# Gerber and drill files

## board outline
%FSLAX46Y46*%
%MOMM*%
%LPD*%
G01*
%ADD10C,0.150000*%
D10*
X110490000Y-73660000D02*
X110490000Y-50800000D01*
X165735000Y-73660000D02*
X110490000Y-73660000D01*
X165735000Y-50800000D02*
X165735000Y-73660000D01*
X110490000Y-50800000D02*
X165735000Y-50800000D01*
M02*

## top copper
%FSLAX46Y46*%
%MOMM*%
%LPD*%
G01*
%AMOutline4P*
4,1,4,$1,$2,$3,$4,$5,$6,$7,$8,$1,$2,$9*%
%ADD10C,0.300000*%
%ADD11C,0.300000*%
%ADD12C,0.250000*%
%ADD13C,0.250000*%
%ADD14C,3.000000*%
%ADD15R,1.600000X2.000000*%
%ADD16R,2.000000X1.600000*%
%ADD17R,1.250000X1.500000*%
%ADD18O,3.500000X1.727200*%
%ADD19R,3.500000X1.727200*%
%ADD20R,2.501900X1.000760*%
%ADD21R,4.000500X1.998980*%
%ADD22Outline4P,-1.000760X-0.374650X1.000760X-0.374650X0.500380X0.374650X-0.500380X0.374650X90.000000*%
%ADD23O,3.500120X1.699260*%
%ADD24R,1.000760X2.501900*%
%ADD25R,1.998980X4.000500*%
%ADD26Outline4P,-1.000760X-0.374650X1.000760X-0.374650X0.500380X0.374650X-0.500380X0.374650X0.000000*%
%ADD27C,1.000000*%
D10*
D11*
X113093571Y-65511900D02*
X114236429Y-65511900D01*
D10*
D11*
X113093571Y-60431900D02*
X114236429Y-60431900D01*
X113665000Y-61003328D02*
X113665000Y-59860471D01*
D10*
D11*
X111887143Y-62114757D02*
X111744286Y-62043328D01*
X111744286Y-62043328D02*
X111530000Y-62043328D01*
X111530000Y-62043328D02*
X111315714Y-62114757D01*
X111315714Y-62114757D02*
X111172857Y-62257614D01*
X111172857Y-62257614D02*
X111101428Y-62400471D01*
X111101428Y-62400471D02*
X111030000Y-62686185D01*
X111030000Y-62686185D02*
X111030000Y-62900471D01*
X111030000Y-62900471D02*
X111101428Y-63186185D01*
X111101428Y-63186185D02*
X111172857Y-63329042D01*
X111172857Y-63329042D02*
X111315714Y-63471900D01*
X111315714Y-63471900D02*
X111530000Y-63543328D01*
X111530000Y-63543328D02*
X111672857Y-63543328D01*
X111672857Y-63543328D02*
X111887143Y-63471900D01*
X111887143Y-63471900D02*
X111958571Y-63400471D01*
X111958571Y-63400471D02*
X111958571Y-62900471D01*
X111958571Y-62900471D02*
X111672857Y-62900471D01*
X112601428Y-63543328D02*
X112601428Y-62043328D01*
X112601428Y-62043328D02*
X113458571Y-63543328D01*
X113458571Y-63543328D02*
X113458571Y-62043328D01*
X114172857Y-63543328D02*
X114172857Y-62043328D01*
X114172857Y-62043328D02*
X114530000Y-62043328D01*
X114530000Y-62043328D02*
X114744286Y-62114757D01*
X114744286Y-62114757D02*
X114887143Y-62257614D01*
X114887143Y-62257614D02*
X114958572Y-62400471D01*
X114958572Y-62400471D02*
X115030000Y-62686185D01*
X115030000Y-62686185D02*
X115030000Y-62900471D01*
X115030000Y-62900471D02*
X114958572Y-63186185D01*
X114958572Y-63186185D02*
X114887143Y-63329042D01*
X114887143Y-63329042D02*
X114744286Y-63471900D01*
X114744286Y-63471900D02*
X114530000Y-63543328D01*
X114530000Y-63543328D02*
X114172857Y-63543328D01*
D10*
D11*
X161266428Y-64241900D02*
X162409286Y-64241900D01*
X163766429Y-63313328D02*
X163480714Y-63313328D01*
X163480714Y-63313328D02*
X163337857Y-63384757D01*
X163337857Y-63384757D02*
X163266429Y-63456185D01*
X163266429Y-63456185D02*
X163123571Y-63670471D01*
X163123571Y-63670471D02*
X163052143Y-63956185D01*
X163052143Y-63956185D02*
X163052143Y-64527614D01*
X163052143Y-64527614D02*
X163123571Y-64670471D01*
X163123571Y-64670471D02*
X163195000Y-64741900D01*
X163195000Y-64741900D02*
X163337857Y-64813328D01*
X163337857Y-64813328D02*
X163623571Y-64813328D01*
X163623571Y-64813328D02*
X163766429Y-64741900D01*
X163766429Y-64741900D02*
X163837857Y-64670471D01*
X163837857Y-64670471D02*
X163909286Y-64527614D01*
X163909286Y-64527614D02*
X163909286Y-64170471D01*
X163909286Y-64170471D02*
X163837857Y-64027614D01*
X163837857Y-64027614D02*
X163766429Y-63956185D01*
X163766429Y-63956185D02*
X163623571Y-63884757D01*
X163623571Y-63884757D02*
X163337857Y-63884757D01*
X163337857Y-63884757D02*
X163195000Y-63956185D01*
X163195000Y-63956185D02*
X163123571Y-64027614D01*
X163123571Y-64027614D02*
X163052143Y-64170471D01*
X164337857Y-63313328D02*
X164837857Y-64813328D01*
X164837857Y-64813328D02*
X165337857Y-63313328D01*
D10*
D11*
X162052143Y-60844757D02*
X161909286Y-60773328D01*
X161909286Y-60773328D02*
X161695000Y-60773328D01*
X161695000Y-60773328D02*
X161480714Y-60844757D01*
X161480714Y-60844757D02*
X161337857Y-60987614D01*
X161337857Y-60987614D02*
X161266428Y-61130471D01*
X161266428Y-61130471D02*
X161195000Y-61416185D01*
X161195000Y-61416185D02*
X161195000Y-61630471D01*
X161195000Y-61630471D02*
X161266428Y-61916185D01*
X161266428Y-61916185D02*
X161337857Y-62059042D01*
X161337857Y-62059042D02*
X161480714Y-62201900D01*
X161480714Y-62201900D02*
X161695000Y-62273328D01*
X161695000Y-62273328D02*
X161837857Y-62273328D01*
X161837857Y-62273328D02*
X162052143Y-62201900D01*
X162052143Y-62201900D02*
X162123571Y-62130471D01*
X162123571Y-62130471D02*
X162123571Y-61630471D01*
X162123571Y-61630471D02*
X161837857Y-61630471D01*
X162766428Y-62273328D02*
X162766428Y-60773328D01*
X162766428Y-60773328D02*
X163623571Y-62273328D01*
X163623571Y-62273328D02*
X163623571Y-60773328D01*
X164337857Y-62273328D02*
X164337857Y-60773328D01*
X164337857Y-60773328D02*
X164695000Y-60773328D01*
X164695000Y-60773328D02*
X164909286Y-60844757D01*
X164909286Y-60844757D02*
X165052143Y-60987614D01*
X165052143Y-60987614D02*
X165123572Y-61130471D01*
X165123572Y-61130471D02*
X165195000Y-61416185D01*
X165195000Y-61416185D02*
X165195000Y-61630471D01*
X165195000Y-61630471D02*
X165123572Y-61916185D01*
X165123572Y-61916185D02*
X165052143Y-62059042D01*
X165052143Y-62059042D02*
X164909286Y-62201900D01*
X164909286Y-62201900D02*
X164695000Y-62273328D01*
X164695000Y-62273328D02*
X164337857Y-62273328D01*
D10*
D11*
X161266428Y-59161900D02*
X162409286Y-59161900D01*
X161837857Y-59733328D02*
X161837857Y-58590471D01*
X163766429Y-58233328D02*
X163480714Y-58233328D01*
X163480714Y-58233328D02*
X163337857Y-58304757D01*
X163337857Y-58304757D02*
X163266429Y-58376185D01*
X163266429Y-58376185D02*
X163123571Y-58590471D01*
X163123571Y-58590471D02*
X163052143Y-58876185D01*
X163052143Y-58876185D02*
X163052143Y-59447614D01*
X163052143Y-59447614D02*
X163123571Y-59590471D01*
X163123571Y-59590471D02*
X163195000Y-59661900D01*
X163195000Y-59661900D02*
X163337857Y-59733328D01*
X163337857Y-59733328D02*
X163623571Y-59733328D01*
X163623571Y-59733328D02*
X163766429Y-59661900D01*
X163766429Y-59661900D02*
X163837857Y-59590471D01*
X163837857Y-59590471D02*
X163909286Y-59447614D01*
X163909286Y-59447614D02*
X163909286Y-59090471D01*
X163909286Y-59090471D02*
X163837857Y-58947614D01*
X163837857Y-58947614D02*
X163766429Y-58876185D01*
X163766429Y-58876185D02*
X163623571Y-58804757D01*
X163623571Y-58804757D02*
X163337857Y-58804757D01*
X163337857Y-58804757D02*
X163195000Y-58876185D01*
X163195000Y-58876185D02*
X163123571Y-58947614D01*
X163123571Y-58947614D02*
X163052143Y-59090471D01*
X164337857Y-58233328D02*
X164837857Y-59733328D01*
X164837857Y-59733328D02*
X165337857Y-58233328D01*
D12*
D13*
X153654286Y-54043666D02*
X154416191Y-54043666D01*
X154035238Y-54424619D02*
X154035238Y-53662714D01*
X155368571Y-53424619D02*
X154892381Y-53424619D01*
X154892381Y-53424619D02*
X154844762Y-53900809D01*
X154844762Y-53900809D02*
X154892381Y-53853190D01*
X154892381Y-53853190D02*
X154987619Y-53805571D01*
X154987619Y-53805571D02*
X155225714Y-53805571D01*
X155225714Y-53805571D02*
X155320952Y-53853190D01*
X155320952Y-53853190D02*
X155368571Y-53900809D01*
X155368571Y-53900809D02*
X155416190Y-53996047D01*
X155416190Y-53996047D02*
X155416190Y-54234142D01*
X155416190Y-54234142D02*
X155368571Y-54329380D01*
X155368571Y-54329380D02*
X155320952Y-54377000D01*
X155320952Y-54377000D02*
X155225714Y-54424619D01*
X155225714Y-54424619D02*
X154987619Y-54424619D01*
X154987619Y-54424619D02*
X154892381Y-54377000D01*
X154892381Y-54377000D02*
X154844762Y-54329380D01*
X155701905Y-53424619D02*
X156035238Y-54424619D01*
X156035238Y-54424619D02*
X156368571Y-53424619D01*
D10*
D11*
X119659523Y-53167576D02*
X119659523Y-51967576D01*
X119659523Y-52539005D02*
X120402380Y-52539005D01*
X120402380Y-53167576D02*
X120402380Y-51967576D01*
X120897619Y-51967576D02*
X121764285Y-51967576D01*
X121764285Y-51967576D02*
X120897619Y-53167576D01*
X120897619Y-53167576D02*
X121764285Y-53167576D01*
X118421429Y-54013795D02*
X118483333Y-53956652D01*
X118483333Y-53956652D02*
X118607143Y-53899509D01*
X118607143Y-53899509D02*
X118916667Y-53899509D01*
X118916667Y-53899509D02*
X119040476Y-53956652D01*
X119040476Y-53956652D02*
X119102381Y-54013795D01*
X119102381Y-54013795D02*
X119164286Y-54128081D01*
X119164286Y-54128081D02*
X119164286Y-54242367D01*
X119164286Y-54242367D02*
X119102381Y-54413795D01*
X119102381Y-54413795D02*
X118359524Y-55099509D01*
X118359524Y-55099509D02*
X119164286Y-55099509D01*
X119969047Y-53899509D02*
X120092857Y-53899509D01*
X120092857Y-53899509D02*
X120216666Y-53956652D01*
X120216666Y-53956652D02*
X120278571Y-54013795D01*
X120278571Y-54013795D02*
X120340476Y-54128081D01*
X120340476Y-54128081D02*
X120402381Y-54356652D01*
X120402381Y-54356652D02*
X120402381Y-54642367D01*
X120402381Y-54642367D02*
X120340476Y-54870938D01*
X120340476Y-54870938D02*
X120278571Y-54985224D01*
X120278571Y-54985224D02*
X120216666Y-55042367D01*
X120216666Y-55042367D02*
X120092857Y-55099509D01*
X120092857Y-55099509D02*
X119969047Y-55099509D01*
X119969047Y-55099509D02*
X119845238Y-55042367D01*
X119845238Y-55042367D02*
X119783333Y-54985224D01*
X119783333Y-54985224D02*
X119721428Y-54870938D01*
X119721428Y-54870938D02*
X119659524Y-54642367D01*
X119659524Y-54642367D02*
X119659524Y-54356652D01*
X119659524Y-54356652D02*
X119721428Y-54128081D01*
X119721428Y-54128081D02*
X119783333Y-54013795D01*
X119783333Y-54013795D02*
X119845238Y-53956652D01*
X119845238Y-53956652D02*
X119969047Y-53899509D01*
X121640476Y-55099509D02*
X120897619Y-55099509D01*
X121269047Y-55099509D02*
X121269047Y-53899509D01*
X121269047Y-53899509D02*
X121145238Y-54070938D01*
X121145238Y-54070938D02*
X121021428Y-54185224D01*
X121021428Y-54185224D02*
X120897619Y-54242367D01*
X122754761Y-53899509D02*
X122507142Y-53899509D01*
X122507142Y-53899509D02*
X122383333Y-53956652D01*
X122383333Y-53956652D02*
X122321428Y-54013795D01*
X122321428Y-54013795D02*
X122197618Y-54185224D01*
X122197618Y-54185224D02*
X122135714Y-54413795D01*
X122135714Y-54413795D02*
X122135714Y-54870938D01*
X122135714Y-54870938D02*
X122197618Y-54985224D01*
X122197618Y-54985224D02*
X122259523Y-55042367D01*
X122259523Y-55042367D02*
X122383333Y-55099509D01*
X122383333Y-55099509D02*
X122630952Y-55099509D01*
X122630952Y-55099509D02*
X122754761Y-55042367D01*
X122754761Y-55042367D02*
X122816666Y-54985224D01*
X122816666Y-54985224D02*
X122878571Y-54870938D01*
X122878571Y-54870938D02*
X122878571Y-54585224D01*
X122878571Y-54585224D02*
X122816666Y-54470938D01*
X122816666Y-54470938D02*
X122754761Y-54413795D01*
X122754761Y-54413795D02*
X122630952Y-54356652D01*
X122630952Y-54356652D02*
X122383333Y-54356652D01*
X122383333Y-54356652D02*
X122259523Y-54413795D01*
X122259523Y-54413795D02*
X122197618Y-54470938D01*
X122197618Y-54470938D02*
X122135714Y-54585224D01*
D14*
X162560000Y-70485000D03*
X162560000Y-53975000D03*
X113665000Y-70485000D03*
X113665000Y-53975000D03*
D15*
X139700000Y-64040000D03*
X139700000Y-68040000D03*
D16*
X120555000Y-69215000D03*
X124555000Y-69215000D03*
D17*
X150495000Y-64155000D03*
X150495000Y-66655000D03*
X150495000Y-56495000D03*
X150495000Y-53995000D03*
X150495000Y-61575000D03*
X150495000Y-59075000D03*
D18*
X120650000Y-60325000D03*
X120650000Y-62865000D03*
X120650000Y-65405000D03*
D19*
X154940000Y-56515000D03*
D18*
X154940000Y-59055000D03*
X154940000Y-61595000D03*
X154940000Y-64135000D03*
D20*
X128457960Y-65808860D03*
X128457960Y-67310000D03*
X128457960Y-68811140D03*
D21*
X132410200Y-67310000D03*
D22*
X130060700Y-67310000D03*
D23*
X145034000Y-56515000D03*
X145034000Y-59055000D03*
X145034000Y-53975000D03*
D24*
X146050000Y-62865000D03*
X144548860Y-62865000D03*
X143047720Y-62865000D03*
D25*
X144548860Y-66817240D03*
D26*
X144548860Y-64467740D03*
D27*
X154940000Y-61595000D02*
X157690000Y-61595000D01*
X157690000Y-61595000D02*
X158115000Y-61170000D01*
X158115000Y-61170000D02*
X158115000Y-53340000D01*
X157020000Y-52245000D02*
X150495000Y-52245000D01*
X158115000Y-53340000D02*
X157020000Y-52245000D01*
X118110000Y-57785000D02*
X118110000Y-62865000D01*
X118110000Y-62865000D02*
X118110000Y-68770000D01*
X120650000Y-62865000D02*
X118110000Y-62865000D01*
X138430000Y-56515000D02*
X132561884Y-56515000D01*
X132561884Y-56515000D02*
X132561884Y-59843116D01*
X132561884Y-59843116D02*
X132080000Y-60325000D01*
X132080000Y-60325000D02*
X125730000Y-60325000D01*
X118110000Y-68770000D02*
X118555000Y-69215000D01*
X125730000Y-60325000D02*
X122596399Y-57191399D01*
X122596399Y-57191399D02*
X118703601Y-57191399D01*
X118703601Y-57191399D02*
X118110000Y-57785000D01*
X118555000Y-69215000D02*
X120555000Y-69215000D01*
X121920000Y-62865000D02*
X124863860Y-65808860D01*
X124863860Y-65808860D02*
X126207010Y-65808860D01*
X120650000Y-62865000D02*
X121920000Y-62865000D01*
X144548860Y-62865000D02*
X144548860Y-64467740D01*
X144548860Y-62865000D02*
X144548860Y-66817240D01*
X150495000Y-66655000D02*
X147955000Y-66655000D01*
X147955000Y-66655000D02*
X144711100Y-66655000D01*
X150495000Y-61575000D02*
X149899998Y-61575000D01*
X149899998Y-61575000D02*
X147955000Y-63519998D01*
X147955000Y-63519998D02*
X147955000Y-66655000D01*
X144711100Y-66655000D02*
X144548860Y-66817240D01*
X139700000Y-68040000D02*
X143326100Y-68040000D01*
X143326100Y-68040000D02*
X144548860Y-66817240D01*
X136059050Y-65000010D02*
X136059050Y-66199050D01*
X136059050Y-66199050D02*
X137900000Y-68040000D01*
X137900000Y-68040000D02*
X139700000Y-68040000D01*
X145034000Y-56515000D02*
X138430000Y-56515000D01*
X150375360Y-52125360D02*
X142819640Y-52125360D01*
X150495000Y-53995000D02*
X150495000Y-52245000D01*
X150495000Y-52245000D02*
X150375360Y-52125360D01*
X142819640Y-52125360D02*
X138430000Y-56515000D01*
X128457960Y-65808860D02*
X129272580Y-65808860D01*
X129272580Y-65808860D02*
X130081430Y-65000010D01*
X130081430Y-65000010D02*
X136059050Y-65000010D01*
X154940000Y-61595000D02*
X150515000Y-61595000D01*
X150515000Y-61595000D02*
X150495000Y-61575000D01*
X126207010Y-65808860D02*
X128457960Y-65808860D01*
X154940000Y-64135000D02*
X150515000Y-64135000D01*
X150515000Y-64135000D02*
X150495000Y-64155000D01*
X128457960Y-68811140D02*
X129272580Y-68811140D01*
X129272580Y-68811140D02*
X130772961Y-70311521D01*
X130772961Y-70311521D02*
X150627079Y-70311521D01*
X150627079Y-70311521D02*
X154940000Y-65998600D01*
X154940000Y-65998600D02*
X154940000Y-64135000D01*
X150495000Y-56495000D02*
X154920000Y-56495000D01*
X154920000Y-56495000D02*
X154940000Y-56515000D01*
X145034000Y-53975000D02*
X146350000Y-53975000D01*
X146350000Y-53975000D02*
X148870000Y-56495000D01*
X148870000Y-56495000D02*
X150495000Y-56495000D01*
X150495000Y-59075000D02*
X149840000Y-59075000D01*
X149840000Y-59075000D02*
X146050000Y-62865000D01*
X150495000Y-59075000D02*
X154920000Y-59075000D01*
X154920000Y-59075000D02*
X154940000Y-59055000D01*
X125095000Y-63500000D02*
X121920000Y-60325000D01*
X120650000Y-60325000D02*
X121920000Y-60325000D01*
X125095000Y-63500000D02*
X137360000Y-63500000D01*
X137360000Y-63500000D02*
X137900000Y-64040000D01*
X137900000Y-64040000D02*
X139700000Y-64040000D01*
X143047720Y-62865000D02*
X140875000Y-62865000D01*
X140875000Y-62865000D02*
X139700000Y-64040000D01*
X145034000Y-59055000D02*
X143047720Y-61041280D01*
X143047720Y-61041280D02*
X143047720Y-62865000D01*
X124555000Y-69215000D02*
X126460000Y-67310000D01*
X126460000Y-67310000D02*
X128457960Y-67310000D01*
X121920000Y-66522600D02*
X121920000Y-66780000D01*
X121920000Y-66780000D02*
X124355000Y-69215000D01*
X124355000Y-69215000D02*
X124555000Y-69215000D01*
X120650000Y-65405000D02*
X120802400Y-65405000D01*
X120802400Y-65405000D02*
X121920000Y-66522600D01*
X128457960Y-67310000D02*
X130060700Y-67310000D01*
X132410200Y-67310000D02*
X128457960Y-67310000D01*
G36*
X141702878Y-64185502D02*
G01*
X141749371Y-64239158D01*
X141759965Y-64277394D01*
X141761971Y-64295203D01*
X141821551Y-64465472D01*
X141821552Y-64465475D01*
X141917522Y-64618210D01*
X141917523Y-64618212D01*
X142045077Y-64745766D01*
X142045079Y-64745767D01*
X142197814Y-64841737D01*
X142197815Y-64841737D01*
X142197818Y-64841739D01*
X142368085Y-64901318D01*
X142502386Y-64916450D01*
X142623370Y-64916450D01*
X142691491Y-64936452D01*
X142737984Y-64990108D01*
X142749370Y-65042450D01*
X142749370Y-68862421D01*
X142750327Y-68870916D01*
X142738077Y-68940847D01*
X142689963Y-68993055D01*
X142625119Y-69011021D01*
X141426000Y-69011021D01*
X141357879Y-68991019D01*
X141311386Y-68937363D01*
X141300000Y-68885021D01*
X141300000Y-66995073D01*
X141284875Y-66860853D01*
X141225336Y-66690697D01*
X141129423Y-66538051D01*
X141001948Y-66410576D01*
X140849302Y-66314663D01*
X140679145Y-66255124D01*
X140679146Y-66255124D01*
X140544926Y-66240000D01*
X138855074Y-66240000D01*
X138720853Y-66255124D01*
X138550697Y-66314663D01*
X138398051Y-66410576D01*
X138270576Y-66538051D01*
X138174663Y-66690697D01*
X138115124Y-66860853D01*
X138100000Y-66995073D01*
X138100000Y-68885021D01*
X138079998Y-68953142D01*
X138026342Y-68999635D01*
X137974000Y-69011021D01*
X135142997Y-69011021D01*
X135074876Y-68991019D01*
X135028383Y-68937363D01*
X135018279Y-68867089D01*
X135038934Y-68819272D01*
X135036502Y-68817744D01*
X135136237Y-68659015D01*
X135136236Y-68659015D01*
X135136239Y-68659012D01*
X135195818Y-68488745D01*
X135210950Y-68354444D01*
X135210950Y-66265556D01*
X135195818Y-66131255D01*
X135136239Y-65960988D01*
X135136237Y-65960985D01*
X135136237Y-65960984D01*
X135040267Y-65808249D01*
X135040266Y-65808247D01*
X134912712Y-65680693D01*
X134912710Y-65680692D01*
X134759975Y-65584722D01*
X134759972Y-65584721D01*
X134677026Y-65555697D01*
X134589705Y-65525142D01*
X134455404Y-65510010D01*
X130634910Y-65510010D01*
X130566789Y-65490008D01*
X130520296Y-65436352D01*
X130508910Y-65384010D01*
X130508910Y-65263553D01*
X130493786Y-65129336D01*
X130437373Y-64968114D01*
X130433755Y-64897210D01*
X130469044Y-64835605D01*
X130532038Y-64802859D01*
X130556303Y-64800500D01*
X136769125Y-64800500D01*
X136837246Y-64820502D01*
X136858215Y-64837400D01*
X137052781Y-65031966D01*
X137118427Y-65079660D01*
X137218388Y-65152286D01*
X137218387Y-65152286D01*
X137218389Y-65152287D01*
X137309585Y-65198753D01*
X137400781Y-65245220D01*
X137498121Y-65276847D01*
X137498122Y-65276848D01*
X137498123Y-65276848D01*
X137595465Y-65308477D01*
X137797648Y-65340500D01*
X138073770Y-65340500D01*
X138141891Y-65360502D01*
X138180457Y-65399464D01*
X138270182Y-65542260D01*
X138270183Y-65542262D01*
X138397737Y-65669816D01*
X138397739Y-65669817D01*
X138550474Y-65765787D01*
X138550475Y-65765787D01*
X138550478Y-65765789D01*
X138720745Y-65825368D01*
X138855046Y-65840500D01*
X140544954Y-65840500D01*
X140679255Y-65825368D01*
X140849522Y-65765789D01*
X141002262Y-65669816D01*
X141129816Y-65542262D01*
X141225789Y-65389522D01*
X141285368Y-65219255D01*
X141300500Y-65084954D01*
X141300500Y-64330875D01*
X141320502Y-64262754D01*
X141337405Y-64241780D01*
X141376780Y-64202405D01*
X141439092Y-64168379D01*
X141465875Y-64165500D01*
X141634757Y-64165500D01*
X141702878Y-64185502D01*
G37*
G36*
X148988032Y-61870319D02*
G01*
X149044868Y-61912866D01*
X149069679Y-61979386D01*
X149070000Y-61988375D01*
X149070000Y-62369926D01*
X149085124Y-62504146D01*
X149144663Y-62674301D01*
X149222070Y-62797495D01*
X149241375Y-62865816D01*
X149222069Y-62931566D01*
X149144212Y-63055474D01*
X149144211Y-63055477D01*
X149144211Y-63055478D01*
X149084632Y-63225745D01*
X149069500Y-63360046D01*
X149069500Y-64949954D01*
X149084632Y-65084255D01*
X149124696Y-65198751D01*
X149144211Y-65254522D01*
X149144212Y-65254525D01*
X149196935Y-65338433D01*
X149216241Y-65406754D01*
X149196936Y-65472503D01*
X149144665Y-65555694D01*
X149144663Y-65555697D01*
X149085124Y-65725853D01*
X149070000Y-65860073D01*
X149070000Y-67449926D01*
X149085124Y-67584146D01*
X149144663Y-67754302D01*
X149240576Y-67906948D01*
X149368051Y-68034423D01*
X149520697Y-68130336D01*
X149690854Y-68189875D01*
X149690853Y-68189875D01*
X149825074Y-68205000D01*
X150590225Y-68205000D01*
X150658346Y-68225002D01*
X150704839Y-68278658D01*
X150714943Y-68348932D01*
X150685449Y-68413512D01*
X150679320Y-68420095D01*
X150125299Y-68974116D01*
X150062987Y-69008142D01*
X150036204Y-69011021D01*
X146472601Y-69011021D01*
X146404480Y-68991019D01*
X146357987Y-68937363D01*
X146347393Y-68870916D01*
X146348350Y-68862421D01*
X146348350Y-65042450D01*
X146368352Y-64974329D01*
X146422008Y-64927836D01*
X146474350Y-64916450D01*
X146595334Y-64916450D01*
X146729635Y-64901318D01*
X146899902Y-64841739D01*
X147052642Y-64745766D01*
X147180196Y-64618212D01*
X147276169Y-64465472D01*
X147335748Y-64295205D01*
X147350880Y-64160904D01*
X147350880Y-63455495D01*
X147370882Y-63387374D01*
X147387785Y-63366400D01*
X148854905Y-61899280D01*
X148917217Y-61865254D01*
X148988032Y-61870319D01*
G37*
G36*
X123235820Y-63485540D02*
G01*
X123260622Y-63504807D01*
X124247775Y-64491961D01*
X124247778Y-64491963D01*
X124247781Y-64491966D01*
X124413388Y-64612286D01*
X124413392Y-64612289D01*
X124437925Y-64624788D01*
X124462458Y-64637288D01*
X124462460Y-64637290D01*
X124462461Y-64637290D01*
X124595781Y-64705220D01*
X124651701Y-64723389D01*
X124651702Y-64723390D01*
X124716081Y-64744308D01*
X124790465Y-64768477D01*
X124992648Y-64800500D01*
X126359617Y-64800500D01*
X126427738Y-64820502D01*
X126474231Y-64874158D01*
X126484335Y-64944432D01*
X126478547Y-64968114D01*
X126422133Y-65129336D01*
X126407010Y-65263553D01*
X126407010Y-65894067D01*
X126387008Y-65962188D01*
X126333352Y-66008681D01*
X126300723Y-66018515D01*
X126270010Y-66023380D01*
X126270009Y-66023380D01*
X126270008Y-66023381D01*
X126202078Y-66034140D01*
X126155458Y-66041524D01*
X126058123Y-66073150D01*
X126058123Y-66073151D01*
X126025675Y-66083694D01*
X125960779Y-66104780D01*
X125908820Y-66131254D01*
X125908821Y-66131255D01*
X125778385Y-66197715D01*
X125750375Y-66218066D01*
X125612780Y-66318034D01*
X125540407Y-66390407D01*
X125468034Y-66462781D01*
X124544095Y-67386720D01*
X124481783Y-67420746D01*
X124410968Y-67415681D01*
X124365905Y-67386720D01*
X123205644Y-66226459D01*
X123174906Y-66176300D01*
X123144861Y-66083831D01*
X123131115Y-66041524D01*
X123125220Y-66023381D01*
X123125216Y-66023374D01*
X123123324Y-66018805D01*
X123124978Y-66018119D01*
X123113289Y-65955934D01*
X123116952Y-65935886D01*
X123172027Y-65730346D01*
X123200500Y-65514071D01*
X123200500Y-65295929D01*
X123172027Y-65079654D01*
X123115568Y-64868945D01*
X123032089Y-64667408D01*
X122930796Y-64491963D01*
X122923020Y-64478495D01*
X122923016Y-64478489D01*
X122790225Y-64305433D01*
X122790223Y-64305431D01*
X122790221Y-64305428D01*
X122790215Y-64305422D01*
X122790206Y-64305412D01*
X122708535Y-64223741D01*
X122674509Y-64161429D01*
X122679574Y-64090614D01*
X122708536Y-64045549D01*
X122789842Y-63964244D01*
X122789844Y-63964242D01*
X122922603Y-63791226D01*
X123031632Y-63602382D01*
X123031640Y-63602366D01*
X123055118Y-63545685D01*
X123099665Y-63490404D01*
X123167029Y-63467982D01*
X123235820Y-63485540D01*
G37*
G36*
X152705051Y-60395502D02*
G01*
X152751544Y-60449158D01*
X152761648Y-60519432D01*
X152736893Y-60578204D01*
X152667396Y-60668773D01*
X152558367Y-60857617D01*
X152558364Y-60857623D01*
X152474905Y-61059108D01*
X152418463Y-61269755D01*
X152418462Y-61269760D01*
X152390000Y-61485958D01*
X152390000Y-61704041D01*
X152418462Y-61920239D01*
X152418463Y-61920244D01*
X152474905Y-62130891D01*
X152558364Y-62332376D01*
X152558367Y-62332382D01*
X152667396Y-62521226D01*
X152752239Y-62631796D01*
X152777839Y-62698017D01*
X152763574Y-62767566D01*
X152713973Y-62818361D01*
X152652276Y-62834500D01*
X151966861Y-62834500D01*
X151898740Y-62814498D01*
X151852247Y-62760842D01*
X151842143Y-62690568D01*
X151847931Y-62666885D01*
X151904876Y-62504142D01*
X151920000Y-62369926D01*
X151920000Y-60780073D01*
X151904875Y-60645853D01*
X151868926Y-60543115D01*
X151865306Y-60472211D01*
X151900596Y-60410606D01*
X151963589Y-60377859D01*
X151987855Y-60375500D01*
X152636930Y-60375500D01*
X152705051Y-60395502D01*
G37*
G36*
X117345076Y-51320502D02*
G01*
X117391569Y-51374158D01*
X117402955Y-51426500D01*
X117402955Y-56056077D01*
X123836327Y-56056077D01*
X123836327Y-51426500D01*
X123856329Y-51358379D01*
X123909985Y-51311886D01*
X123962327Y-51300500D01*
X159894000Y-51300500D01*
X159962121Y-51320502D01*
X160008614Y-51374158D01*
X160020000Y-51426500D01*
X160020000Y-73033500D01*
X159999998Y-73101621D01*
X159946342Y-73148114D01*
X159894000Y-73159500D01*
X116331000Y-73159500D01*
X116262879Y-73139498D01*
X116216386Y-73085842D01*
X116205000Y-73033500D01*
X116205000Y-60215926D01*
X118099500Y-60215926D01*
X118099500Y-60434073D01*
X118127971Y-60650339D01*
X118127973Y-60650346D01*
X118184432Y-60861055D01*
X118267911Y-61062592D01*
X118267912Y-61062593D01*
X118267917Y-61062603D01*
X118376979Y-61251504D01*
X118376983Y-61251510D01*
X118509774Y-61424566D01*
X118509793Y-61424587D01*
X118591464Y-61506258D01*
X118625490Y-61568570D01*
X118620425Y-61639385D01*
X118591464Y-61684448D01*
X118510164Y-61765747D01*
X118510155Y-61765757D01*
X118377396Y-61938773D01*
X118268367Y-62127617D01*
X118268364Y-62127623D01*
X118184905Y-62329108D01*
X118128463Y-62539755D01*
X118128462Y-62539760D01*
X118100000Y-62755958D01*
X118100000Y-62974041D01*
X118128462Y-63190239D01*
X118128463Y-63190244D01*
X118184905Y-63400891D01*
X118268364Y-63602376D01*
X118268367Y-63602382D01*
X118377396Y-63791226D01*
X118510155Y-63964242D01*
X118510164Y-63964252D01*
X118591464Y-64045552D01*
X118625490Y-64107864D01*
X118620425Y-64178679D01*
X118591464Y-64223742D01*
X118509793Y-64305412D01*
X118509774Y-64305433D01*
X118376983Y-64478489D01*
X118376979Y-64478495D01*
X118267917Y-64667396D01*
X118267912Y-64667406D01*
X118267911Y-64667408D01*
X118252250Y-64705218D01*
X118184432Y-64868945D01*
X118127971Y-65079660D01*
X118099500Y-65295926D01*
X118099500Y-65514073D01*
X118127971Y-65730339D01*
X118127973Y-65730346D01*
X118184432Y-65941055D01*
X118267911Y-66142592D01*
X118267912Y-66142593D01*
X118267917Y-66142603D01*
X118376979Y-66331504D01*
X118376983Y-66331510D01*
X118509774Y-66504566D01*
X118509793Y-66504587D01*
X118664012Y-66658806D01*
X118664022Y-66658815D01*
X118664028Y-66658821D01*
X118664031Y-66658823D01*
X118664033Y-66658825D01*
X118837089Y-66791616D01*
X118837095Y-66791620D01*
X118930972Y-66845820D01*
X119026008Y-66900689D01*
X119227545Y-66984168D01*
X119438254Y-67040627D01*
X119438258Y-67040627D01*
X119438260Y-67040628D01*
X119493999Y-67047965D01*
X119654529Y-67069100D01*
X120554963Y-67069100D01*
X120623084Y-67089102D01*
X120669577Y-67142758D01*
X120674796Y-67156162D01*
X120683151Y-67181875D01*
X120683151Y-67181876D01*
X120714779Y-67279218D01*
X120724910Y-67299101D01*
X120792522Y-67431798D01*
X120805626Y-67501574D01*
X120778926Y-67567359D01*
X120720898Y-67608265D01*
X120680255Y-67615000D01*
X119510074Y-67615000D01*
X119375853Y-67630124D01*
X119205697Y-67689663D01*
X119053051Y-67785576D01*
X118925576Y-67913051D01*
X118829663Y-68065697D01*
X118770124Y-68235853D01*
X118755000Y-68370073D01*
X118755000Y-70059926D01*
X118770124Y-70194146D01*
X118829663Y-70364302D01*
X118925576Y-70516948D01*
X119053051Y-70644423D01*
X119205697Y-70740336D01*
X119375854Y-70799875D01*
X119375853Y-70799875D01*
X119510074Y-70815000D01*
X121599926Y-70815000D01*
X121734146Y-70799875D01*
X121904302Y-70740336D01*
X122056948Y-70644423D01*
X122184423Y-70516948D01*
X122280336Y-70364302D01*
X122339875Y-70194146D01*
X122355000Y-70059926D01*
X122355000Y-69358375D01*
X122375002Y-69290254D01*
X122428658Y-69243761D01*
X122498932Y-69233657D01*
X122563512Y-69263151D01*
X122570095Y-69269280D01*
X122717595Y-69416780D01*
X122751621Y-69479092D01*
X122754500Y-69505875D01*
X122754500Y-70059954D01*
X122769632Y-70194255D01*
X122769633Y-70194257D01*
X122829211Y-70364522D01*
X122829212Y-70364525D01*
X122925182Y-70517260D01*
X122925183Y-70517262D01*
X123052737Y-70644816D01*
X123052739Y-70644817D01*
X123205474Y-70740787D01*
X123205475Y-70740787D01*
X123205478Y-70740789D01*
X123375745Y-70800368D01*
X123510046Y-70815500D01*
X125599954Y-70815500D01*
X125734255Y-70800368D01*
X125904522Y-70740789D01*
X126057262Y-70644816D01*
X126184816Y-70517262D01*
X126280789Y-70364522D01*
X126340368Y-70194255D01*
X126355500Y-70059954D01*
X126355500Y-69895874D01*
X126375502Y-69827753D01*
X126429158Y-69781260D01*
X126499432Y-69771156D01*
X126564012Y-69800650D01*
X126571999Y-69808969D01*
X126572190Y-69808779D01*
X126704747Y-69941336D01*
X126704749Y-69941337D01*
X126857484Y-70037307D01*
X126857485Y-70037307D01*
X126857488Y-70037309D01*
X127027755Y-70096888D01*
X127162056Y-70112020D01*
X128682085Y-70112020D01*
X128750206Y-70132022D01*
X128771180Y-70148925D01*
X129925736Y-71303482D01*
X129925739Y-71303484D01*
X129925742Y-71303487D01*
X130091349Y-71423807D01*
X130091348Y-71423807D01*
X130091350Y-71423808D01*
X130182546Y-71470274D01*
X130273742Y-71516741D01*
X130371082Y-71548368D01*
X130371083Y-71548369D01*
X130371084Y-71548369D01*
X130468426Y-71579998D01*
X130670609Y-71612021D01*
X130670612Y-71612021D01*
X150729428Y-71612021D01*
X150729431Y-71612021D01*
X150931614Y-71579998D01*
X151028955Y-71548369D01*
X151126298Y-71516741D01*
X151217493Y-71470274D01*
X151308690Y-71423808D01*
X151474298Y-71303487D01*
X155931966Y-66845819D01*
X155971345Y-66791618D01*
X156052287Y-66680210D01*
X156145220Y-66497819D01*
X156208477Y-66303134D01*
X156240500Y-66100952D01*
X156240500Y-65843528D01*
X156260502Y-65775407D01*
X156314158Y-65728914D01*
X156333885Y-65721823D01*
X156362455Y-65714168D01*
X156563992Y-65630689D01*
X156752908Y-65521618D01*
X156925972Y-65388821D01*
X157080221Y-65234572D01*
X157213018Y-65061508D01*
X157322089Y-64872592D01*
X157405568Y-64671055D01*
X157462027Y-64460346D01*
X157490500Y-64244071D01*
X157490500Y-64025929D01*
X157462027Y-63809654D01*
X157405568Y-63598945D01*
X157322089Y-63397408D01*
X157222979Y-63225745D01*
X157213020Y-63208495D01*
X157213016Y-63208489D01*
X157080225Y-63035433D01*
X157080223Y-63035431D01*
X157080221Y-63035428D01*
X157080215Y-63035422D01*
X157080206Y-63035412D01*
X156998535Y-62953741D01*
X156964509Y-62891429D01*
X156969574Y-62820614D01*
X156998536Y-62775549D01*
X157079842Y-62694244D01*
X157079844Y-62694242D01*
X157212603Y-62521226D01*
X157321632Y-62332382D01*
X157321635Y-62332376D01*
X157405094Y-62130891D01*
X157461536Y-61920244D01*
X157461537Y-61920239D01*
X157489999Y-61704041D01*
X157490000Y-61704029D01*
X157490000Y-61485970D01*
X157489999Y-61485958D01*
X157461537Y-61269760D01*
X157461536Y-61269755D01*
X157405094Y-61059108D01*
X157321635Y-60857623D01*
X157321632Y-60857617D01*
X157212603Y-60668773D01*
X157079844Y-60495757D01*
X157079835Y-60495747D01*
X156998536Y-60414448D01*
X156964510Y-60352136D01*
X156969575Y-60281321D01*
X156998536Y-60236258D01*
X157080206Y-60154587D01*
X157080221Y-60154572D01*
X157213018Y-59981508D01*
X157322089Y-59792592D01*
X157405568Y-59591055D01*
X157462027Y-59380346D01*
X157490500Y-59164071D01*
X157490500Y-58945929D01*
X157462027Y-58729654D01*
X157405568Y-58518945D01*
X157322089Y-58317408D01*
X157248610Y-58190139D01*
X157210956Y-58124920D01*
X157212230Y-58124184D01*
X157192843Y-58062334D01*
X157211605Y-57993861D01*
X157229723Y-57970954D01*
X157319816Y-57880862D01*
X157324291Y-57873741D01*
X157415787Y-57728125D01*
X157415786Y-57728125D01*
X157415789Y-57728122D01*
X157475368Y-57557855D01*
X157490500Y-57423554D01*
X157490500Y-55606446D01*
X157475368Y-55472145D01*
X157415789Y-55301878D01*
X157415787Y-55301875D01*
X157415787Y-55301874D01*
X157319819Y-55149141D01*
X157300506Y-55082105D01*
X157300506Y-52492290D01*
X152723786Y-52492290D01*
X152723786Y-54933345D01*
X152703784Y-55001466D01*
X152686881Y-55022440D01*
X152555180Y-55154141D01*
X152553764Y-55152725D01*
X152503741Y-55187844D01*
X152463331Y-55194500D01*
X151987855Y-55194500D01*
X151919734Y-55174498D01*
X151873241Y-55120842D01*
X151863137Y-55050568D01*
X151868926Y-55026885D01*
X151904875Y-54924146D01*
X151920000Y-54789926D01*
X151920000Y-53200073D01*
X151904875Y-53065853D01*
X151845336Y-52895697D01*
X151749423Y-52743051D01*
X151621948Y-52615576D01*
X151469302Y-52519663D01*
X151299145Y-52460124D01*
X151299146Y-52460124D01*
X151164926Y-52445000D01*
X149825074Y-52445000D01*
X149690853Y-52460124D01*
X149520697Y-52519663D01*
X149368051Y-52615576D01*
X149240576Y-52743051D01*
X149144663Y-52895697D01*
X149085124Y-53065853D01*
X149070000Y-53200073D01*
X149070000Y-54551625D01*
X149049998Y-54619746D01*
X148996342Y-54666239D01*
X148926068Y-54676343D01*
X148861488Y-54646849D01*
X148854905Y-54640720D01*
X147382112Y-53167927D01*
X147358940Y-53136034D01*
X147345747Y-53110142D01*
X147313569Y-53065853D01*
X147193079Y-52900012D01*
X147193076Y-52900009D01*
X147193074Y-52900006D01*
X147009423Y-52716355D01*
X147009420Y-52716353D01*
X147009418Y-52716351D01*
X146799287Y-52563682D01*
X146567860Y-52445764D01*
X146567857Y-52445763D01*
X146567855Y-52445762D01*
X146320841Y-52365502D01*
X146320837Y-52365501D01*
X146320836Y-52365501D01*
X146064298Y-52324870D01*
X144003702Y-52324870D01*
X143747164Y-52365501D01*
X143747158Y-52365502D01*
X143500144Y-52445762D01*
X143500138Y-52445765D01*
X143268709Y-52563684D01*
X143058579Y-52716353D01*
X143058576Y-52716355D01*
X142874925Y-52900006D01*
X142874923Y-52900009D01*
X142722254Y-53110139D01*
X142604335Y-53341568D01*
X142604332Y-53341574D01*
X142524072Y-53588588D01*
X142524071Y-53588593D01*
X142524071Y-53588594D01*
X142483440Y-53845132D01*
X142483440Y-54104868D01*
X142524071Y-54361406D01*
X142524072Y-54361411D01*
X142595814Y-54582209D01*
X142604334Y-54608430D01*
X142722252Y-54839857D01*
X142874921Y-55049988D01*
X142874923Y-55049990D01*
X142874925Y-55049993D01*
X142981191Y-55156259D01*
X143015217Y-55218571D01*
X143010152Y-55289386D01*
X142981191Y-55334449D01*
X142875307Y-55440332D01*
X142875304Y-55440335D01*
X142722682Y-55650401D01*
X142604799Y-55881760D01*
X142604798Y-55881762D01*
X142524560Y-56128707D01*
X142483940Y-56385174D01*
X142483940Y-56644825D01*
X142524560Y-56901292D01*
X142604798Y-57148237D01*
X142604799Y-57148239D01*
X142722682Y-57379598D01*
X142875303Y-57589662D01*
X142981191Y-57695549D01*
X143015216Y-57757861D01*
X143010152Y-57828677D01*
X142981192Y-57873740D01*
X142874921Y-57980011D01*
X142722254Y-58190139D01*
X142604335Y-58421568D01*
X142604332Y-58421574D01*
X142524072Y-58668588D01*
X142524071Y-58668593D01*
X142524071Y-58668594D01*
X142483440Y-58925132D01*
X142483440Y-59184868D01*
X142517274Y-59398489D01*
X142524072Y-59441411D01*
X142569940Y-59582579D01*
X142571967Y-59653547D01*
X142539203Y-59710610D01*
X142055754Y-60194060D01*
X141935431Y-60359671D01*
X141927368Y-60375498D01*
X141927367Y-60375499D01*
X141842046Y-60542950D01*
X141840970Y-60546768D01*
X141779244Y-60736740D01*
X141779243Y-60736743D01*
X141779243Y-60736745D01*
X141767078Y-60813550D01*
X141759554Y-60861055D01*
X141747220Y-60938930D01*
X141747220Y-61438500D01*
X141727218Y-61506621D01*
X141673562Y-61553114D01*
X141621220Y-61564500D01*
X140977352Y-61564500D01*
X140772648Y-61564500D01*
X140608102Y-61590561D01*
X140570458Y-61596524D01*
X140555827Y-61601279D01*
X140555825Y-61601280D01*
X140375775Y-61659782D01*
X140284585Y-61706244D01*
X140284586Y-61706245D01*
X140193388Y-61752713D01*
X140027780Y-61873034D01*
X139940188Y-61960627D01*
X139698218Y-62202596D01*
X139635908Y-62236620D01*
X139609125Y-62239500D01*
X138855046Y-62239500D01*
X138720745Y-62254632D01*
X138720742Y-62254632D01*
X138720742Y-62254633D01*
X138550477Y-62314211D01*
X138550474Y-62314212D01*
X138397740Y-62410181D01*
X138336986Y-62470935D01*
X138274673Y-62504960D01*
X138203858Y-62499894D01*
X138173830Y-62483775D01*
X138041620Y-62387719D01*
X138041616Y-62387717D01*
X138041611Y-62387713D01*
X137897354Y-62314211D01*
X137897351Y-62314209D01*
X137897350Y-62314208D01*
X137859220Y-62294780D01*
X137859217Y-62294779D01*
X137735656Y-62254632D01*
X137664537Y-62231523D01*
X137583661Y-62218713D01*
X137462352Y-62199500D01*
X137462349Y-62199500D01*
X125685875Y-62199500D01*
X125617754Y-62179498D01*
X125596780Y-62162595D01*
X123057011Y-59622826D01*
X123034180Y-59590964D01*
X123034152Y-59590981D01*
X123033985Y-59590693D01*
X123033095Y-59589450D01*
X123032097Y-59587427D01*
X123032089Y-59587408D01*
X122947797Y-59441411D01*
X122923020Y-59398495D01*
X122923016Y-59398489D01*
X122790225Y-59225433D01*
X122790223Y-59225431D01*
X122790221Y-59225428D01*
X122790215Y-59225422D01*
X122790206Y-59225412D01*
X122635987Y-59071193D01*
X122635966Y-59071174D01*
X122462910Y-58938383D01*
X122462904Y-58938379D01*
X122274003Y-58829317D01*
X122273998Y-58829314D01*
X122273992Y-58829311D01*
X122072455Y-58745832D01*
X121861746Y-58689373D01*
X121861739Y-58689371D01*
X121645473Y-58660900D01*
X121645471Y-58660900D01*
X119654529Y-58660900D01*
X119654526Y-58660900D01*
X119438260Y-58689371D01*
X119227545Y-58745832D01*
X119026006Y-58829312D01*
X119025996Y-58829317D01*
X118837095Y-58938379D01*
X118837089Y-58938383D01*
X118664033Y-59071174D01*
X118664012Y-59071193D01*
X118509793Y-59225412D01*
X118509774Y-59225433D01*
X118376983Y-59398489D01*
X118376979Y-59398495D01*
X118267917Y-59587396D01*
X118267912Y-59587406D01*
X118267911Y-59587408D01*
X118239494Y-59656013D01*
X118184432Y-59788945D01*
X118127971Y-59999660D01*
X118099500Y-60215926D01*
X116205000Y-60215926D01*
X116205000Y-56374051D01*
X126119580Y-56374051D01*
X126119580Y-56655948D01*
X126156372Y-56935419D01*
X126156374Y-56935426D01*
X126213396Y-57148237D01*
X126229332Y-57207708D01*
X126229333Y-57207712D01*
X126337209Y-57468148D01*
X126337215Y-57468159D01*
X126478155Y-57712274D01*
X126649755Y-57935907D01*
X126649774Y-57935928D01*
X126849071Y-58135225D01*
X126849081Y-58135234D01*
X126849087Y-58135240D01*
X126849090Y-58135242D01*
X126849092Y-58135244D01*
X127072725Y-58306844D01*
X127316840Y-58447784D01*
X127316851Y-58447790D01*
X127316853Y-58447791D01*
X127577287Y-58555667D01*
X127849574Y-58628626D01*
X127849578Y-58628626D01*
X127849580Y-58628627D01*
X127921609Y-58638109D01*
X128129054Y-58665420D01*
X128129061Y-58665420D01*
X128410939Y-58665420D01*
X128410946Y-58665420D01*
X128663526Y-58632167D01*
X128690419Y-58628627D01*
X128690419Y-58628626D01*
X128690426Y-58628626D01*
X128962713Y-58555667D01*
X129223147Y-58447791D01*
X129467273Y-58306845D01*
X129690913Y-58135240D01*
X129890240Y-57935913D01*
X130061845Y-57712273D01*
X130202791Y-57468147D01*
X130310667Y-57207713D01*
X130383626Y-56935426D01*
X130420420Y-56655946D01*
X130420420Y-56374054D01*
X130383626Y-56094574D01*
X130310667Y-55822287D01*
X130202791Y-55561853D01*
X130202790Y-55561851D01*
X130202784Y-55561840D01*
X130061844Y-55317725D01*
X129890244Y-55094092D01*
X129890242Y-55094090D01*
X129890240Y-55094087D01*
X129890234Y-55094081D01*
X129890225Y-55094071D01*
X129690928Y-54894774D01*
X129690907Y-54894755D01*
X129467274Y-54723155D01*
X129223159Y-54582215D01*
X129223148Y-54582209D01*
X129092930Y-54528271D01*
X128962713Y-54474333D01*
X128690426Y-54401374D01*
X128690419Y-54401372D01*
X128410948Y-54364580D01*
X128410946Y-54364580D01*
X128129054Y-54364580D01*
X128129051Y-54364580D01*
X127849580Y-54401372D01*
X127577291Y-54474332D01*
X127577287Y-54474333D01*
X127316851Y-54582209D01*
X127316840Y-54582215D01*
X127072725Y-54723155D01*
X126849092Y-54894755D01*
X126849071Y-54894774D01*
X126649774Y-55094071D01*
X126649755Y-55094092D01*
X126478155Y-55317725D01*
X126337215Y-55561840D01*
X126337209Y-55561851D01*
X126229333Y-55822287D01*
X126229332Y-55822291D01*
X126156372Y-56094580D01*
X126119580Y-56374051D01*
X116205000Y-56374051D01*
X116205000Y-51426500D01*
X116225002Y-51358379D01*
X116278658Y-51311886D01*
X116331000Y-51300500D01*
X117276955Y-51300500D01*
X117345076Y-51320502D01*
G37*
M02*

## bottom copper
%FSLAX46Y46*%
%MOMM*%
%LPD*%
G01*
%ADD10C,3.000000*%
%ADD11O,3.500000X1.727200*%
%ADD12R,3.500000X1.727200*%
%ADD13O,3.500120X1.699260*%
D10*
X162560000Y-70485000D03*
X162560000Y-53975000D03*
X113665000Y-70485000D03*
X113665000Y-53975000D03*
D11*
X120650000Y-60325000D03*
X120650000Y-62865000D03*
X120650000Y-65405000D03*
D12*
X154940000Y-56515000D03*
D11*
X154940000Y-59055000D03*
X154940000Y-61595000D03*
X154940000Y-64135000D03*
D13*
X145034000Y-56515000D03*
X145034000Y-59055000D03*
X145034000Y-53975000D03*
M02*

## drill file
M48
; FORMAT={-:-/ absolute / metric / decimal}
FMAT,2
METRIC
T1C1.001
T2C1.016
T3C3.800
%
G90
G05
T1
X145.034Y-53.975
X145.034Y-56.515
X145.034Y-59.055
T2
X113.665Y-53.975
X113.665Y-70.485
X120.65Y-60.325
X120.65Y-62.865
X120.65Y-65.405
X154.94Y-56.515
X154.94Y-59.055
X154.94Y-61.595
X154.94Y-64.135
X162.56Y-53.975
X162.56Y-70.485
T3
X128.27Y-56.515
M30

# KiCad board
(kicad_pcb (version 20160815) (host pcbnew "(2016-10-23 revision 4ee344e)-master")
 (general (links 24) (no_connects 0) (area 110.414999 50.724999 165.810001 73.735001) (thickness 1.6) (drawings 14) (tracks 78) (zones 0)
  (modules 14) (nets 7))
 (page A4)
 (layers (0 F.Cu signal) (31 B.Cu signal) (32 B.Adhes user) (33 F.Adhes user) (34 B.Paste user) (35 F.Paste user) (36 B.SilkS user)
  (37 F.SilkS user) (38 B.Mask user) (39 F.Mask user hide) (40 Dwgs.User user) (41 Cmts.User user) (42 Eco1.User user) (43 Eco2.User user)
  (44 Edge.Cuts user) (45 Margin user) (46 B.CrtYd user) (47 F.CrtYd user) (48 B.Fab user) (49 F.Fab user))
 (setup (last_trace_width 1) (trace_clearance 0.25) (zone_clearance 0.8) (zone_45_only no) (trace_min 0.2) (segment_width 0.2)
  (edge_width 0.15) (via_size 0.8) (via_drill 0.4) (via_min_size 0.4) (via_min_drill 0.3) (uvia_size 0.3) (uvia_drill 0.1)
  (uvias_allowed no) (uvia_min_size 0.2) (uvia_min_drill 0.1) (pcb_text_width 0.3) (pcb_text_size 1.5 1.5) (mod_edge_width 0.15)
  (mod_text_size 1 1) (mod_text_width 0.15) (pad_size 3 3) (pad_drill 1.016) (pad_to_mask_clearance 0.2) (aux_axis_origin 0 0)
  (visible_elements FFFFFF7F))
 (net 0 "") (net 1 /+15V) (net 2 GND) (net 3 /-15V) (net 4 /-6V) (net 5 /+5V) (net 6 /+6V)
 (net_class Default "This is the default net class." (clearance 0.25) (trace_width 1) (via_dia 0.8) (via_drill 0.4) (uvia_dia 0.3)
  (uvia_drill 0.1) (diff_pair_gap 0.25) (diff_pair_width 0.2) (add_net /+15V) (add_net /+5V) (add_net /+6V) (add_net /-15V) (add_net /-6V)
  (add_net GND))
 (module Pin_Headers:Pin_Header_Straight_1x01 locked (layer F.Cu) (at 162.56 70.485)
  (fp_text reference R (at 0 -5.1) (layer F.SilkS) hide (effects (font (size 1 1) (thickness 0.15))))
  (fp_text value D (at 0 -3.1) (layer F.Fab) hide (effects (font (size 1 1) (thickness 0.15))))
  (pad 1 thru_hole circle (at 0 0) (size 3 3) (drill 1.016) (layers *.Cu *.Mask F.SilkS)))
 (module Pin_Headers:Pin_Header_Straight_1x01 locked (layer F.Cu) (at 162.56 53.975)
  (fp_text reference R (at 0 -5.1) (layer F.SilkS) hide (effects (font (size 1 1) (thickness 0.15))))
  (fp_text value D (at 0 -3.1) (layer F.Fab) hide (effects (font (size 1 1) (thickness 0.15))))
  (pad 1 thru_hole circle (at 0 0) (size 3 3) (drill 1.016) (layers *.Cu *.Mask F.SilkS)))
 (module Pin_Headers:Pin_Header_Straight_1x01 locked (layer F.Cu) (at 113.665 70.485)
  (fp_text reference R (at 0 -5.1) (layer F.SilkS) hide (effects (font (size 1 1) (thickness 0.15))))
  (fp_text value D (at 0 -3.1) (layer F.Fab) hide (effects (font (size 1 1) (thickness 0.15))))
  (pad 1 thru_hole circle (at 0 0) (size 3 3) (drill 1.016) (layers *.Cu *.Mask F.SilkS)))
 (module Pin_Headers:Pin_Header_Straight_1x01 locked (layer F.Cu) (at 113.665 53.975)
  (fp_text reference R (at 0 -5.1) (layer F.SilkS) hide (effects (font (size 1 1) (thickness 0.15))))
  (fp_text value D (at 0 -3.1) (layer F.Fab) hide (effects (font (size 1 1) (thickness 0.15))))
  (pad 1 thru_hole circle (at 0 0) (size 3 3) (drill 1.016) (layers *.Cu *.Mask F.SilkS)))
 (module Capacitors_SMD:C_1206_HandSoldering (layer F.Cu) (at 139.7 66.04 270)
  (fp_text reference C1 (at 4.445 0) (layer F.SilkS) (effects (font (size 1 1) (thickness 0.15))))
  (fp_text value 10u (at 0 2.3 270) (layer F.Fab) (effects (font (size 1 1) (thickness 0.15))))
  (pad 1 smd rect (at -2 0 270) (size 2 1.6) (layers F.Cu F.Paste F.Mask) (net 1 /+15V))
  (pad 2 smd rect (at 2 0 270) (size 2 1.6) (layers F.Cu F.Paste F.Mask) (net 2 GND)))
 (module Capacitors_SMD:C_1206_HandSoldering (layer F.Cu) (at 122.555 69.215 180)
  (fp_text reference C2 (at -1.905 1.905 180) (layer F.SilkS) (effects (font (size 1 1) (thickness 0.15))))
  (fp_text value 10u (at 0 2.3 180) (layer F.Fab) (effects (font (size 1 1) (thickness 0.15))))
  (pad 2 smd rect (at 2 0 180) (size 2 1.6) (layers F.Cu F.Paste F.Mask) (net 2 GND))
  (pad 1 smd rect (at -2 0 180) (size 2 1.6) (layers F.Cu F.Paste F.Mask) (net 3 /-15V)))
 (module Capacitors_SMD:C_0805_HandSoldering (layer F.Cu) (at 150.495 65.405 270)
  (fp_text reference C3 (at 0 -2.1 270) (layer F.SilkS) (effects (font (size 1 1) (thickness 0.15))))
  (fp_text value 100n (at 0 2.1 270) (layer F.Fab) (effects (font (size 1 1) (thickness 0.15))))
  (pad 1 smd rect (at -1.25 0 270) (size 1.5 1.25) (layers F.Cu F.Paste F.Mask) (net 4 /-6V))
  (pad 2 smd rect (at 1.25 0 270) (size 1.5 1.25) (layers F.Cu F.Paste F.Mask) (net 2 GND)))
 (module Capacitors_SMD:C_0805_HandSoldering (layer F.Cu) (at 150.495 55.245 90)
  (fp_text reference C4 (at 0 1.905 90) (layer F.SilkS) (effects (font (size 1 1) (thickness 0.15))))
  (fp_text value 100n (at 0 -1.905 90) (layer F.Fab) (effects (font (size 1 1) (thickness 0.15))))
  (pad 1 smd rect (at -1.25 0 90) (size 1.5 1.25) (layers F.Cu F.Paste F.Mask) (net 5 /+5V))
  (pad 2 smd rect (at 1.25 0 90) (size 1.5 1.25) (layers F.Cu F.Paste F.Mask) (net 2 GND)))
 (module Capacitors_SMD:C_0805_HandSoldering (layer F.Cu) (at 150.495 60.325 270)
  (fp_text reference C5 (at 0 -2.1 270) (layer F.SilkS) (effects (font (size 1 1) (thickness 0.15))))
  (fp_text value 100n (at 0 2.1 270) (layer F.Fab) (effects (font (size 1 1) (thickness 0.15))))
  (pad 2 smd rect (at 1.25 0 270) (size 1.5 1.25) (layers F.Cu F.Paste F.Mask) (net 2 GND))
  (pad 1 smd rect (at -1.25 0 270) (size 1.5 1.25) (layers F.Cu F.Paste F.Mask) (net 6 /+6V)))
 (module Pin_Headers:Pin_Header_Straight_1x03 (layer F.Cu) (at 120.65 60.325)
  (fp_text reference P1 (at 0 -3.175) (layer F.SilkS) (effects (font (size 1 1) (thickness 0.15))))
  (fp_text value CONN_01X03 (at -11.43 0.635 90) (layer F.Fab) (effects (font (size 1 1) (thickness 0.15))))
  (pad 1 thru_hole oval (at 0 0) (size 3.5 1.7272) (drill 1.016) (layers *.Cu *.Mask F.SilkS) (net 1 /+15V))
  (pad 2 thru_hole oval (at 0 2.54) (size 3.5 1.7272) (drill 1.016) (layers *.Cu *.Mask F.SilkS) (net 2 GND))
  (pad 3 thru_hole oval (at 0 5.08) (size 3.5 1.7272) (drill 1.016) (layers *.Cu *.Mask F.SilkS) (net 3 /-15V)))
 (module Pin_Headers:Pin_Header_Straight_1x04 (layer F.Cu) (at 154.94 56.515)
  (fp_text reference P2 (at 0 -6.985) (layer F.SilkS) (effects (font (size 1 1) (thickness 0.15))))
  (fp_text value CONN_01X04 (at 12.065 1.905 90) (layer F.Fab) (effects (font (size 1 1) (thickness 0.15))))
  (pad 1 thru_hole rect (at 0 0) (size 3.5 1.7272) (drill 1.016) (layers *.Cu *.Mask F.SilkS) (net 5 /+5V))
  (pad 2 thru_hole oval (at 0 2.54) (size 3.5 1.7272) (drill 1.016) (layers *.Cu *.Mask F.SilkS) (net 6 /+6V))
  (pad 3 thru_hole oval (at 0 5.08) (size 3.5 1.7272) (drill 1.016) (layers *.Cu *.Mask F.SilkS) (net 2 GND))
  (pad 4 thru_hole oval (at 0 7.62) (size 3.5 1.7272) (drill 1.016) (layers *.Cu *.Mask F.SilkS) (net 4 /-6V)))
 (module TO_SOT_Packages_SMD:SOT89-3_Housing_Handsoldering (layer F.Cu) (at 130.81 67.31 270)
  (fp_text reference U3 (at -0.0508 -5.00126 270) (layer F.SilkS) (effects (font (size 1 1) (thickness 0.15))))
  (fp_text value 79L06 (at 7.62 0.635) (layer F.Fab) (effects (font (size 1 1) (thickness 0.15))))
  (pad 1 smd rect (at -1.50114 2.35204 270) (size 1.00076 2.5019) (layers F.Cu F.Paste F.Mask) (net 2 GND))
  (pad 2 smd rect (at 0 2.35204 270) (size 1.00076 2.5019) (layers F.Cu F.Paste F.Mask) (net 3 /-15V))
  (pad 3 smd rect (at 1.50114 2.35204 270) (size 1.00076 2.5019) (layers F.Cu F.Paste F.Mask) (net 4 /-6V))
  (pad 2 smd rect (at 0 -1.6002 270) (size 1.99898 4.0005) (layers F.Cu F.Paste F.Mask) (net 3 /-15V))
  (pad 2 smd trapezoid (at 0 0.7493 90) (size 1.50114 0.7493) (rect_delta 0 0.50038) (layers F.Cu F.Paste F.Mask) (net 3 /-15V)))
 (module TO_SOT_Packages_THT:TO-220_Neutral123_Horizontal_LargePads (layer F.Cu) (at 145.034 56.515 90)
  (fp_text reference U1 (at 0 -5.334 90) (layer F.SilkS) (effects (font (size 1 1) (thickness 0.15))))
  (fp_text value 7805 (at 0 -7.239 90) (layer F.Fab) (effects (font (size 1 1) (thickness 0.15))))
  (pad 2 thru_hole oval (at 0 0 180) (size 3.50012 1.69926) (drill 1.00076) (layers *.Cu *.Mask F.SilkS) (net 2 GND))
  (pad 1 thru_hole oval (at -2.54 0 180) (size 3.50012 1.69926) (drill 1.00076) (layers *.Cu *.Mask F.SilkS) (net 1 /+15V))
  (pad 3 thru_hole oval (at 2.54 0 180) (size 3.50012 1.69926) (drill 1.00076) (layers *.Cu *.Mask F.SilkS) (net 5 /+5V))
  (pad "" np_thru_hole circle (at 0 -16.764 180) (size 3.79984 3.79984) (drill 3.79984) (layers *.Cu *.Mask F.SilkS)))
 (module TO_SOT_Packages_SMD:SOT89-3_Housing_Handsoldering (layer F.Cu) (at 144.54886 65.21704 180)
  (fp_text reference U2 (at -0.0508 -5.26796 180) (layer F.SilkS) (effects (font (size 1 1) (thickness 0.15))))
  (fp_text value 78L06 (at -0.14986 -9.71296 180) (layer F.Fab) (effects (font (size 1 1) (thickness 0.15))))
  (pad 1 smd rect (at -1.50114 2.35204 180) (size 1.00076 2.5019) (layers F.Cu F.Paste F.Mask) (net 6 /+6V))
  (pad 2 smd rect (at 0 2.35204 180) (size 1.00076 2.5019) (layers F.Cu F.Paste F.Mask) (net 2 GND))
  (pad 3 smd rect (at 1.50114 2.35204 180) (size 1.00076 2.5019) (layers F.Cu F.Paste F.Mask) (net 1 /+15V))
  (pad 2 smd rect (at 0 -1.6002 180) (size 1.99898 4.0005) (layers F.Cu F.Paste F.Mask) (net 2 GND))
  (pad 2 smd trapezoid (at 0 0.7493) (size 1.50114 0.7493) (rect_delta 0 0.50038) (layers F.Cu F.Paste F.Mask) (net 2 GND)))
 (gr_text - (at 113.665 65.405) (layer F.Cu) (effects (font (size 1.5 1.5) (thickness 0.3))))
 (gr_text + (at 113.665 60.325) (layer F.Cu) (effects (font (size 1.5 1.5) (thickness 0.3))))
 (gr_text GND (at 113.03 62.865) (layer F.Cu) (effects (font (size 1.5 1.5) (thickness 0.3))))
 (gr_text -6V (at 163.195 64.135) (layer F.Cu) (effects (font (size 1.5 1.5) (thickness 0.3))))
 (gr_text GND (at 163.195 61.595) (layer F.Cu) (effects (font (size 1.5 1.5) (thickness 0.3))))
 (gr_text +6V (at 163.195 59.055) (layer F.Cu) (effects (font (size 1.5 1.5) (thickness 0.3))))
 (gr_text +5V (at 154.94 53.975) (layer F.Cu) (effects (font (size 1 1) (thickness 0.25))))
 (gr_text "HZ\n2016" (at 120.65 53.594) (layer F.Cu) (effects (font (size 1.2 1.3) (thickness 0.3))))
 (gr_line (start 110.49 73.66) (end 110.49 50.8) (layer Edge.Cuts) (width 0.15))
 (gr_line (start 165.735 73.66) (end 110.49 73.66) (layer Edge.Cuts) (width 0.15))
 (gr_line (start 165.735 50.8) (end 165.735 73.66) (layer Edge.Cuts) (width 0.15))
 (gr_line (start 110.49 50.8) (end 165.735 50.8) (layer Edge.Cuts) (width 0.15))
 (segment (start 154.94 61.595) (end 157.69 61.595) (width 1) (layer F.Cu) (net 2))
 (segment (start 157.69 61.595) (end 158.115 61.17) (width 1) (layer F.Cu) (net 2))
 (segment (start 158.115 61.17) (end 158.115 53.34) (width 1) (layer F.Cu) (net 2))
 (segment (start 157.02 52.245) (end 150.495 52.245) (width 1) (layer F.Cu) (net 2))
 (segment (start 158.115 53.34) (end 157.02 52.245) (width 1) (layer F.Cu) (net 2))
 (segment (start 118.11 57.785) (end 118.11 62.865) (width 1) (layer F.Cu) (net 2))
 (segment (start 118.11 62.865) (end 118.11 68.77) (width 1) (layer F.Cu) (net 2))
 (segment (start 120.65 62.865) (end 118.11 62.865) (width 1) (layer F.Cu) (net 2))
 (segment (start 138.43 56.515) (end 132.561884 56.515) (width 1) (layer F.Cu) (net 2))
 (segment (start 132.561884 56.515) (end 132.561884 59.843116) (width 1) (layer F.Cu) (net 2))
 (segment (start 132.561884 59.843116) (end 132.08 60.325) (width 1) (layer F.Cu) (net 2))
 (segment (start 132.08 60.325) (end 125.73 60.325) (width 1) (layer F.Cu) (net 2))
 (segment (start 118.11 68.77) (end 118.555 69.215) (width 1) (layer F.Cu) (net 2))
 (segment (start 125.73 60.325) (end 122.596399 57.191399) (width 1) (layer F.Cu) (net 2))
 (segment (start 122.596399 57.191399) (end 118.703601 57.191399) (width 1) (layer F.Cu) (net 2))
 (segment (start 118.703601 57.191399) (end 118.11 57.785) (width 1) (layer F.Cu) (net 2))
 (segment (start 118.555 69.215) (end 120.555 69.215) (width 1) (layer F.Cu) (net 2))
 (segment (start 121.92 62.865) (end 124.86386 65.80886) (width 1) (layer F.Cu) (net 2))
 (segment (start 124.86386 65.80886) (end 126.20701 65.80886) (width 1) (layer F.Cu) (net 2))
 (segment (start 120.65 62.865) (end 121.92 62.865) (width 1) (layer F.Cu) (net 2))
 (segment (start 144.54886 62.865) (end 144.54886 64.46774) (width 1) (layer F.Cu) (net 2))
 (segment (start 144.54886 62.865) (end 144.54886 66.81724) (width 1) (layer F.Cu) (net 2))
 (segment (start 150.495 66.655) (end 147.955 66.655) (width 1) (layer F.Cu) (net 2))
 (segment (start 147.955 66.655) (end 144.7111 66.655) (width 1) (layer F.Cu) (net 2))
 (segment (start 150.495 61.575) (end 149.899998 61.575) (width 1) (layer F.Cu) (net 2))
 (segment (start 149.899998 61.575) (end 147.955 63.519998) (width 1) (layer F.Cu) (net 2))
 (segment (start 147.955 63.519998) (end 147.955 66.655) (width 1) (layer F.Cu) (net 2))
 (segment (start 144.7111 66.655) (end 144.54886 66.81724) (width 1) (layer F.Cu) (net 2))
 (segment (start 139.7 68.04) (end 143.3261 68.04) (width 1) (layer F.Cu) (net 2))
 (segment (start 143.3261 68.04) (end 144.54886 66.81724) (width 1) (layer F.Cu) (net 2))
 (segment (start 136.05905 65.00001) (end 136.05905 66.19905) (width 1) (layer F.Cu) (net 2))
 (segment (start 136.05905 66.19905) (end 137.9 68.04) (width 1) (layer F.Cu) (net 2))
 (segment (start 137.9 68.04) (end 139.7 68.04) (width 1) (layer F.Cu) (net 2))
 (segment (start 145.034 56.515) (end 138.43 56.515) (width 1) (layer F.Cu) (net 2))
 (segment (start 150.37536 52.12536) (end 142.81964 52.12536) (width 1) (layer F.Cu) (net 2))
 (segment (start 150.495 53.995) (end 150.495 52.245) (width 1) (layer F.Cu) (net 2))
 (segment (start 150.495 52.245) (end 150.37536 52.12536) (width 1) (layer F.Cu) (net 2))
 (segment (start 142.81964 52.12536) (end 138.43 56.515) (width 1) (layer F.Cu) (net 2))
 (segment (start 128.45796 65.80886) (end 129.27258 65.80886) (width 1) (layer F.Cu) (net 2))
 (segment (start 129.27258 65.80886) (end 130.08143 65.00001) (width 1) (layer F.Cu) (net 2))
 (segment (start 130.08143 65.00001) (end 136.05905 65.00001) (width 1) (layer F.Cu) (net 2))
 (segment (start 154.94 61.595) (end 150.515 61.595) (width 1) (layer F.Cu) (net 2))
 (segment (start 150.515 61.595) (end 150.495 61.575) (width 1) (layer F.Cu) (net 2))
 (segment (start 126.20701 65.80886) (end 128.45796 65.80886) (width 1) (layer F.Cu) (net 2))
 (segment (start 154.94 64.135) (end 150.515 64.135) (width 1) (layer F.Cu) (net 4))
 (segment (start 150.515 64.135) (end 150.495 64.155) (width 1) (layer F.Cu) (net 4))
 (segment (start 128.45796 68.81114) (end 129.27258 68.81114) (width 1) (layer F.Cu) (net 4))
 (segment (start 129.27258 68.81114) (end 130.772961 70.311521) (width 1) (layer F.Cu) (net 4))
 (segment (start 130.772961 70.311521) (end 150.627079 70.311521) (width 1) (layer F.Cu) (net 4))
 (segment (start 150.627079 70.311521) (end 154.94 65.9986) (width 1) (layer F.Cu) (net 4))
 (segment (start 154.94 65.9986) (end 154.94 64.135) (width 1) (layer F.Cu) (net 4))
 (segment (start 150.495 56.495) (end 154.92 56.495) (width 1) (layer F.Cu) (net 5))
 (segment (start 154.92 56.495) (end 154.94 56.515) (width 1) (layer F.Cu) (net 5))
 (segment (start 145.034 53.975) (end 146.35 53.975) (width 1) (layer F.Cu) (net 5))
 (segment (start 146.35 53.975) (end 148.87 56.495) (width 1) (layer F.Cu) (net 5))
 (segment (start 148.87 56.495) (end 150.495 56.495) (width 1) (layer F.Cu) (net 5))
 (segment (start 150.495 59.075) (end 149.84 59.075) (width 1) (layer F.Cu) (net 6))
 (segment (start 149.84 59.075) (end 146.05 62.865) (width 1) (layer F.Cu) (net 6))
 (segment (start 150.495 59.075) (end 154.92 59.075) (width 1) (layer F.Cu) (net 6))
 (segment (start 154.92 59.075) (end 154.94 59.055) (width 1) (layer F.Cu) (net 6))
 (segment (start 125.095 63.5) (end 121.92 60.325) (width 1) (layer F.Cu) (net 1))
 (segment (start 120.65 60.325) (end 121.92 60.325) (width 1) (layer F.Cu) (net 1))
 (segment (start 125.095 63.5) (end 137.36 63.5) (width 1) (layer F.Cu) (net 1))
 (segment (start 137.36 63.5) (end 137.9 64.04) (width 1) (layer F.Cu) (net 1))
 (segment (start 137.9 64.04) (end 139.7 64.04) (width 1) (layer F.Cu) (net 1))
 (segment (start 143.04772 62.865) (end 140.875 62.865) (width 1) (layer F.Cu) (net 1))
 (segment (start 140.875 62.865) (end 139.7 64.04) (width 1) (layer F.Cu) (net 1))
 (segment (start 145.034 59.055) (end 143.04772 61.04128) (width 1) (layer F.Cu) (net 1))
 (segment (start 143.04772 61.04128) (end 143.04772 62.865) (width 1) (layer F.Cu) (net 1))
 (segment (start 124.555 69.215) (end 126.46 67.31) (width 1) (layer F.Cu) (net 3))
 (segment (start 126.46 67.31) (end 128.45796 67.31) (width 1) (layer F.Cu) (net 3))
 (segment (start 121.92 66.5226) (end 121.92 66.78) (width 1) (layer F.Cu) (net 3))
 (segment (start 121.92 66.78) (end 124.355 69.215) (width 1) (layer F.Cu) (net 3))
 (segment (start 124.355 69.215) (end 124.555 69.215) (width 1) (layer F.Cu) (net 3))
 (segment (start 120.65 65.405) (end 120.8024 65.405) (width 1) (layer F.Cu) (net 3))
 (segment (start 120.8024 65.405) (end 121.92 66.5226) (width 1) (layer F.Cu) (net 3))
 (segment (start 128.45796 67.31) (end 130.0607 67.31) (width 1) (layer F.Cu) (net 3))
 (segment (start 132.4102 67.31) (end 128.45796 67.31) (width 1) (layer F.Cu) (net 3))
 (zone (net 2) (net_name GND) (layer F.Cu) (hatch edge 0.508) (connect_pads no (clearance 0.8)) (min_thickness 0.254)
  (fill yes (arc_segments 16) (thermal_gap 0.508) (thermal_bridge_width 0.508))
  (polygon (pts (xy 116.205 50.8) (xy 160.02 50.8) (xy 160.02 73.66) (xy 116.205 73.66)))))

